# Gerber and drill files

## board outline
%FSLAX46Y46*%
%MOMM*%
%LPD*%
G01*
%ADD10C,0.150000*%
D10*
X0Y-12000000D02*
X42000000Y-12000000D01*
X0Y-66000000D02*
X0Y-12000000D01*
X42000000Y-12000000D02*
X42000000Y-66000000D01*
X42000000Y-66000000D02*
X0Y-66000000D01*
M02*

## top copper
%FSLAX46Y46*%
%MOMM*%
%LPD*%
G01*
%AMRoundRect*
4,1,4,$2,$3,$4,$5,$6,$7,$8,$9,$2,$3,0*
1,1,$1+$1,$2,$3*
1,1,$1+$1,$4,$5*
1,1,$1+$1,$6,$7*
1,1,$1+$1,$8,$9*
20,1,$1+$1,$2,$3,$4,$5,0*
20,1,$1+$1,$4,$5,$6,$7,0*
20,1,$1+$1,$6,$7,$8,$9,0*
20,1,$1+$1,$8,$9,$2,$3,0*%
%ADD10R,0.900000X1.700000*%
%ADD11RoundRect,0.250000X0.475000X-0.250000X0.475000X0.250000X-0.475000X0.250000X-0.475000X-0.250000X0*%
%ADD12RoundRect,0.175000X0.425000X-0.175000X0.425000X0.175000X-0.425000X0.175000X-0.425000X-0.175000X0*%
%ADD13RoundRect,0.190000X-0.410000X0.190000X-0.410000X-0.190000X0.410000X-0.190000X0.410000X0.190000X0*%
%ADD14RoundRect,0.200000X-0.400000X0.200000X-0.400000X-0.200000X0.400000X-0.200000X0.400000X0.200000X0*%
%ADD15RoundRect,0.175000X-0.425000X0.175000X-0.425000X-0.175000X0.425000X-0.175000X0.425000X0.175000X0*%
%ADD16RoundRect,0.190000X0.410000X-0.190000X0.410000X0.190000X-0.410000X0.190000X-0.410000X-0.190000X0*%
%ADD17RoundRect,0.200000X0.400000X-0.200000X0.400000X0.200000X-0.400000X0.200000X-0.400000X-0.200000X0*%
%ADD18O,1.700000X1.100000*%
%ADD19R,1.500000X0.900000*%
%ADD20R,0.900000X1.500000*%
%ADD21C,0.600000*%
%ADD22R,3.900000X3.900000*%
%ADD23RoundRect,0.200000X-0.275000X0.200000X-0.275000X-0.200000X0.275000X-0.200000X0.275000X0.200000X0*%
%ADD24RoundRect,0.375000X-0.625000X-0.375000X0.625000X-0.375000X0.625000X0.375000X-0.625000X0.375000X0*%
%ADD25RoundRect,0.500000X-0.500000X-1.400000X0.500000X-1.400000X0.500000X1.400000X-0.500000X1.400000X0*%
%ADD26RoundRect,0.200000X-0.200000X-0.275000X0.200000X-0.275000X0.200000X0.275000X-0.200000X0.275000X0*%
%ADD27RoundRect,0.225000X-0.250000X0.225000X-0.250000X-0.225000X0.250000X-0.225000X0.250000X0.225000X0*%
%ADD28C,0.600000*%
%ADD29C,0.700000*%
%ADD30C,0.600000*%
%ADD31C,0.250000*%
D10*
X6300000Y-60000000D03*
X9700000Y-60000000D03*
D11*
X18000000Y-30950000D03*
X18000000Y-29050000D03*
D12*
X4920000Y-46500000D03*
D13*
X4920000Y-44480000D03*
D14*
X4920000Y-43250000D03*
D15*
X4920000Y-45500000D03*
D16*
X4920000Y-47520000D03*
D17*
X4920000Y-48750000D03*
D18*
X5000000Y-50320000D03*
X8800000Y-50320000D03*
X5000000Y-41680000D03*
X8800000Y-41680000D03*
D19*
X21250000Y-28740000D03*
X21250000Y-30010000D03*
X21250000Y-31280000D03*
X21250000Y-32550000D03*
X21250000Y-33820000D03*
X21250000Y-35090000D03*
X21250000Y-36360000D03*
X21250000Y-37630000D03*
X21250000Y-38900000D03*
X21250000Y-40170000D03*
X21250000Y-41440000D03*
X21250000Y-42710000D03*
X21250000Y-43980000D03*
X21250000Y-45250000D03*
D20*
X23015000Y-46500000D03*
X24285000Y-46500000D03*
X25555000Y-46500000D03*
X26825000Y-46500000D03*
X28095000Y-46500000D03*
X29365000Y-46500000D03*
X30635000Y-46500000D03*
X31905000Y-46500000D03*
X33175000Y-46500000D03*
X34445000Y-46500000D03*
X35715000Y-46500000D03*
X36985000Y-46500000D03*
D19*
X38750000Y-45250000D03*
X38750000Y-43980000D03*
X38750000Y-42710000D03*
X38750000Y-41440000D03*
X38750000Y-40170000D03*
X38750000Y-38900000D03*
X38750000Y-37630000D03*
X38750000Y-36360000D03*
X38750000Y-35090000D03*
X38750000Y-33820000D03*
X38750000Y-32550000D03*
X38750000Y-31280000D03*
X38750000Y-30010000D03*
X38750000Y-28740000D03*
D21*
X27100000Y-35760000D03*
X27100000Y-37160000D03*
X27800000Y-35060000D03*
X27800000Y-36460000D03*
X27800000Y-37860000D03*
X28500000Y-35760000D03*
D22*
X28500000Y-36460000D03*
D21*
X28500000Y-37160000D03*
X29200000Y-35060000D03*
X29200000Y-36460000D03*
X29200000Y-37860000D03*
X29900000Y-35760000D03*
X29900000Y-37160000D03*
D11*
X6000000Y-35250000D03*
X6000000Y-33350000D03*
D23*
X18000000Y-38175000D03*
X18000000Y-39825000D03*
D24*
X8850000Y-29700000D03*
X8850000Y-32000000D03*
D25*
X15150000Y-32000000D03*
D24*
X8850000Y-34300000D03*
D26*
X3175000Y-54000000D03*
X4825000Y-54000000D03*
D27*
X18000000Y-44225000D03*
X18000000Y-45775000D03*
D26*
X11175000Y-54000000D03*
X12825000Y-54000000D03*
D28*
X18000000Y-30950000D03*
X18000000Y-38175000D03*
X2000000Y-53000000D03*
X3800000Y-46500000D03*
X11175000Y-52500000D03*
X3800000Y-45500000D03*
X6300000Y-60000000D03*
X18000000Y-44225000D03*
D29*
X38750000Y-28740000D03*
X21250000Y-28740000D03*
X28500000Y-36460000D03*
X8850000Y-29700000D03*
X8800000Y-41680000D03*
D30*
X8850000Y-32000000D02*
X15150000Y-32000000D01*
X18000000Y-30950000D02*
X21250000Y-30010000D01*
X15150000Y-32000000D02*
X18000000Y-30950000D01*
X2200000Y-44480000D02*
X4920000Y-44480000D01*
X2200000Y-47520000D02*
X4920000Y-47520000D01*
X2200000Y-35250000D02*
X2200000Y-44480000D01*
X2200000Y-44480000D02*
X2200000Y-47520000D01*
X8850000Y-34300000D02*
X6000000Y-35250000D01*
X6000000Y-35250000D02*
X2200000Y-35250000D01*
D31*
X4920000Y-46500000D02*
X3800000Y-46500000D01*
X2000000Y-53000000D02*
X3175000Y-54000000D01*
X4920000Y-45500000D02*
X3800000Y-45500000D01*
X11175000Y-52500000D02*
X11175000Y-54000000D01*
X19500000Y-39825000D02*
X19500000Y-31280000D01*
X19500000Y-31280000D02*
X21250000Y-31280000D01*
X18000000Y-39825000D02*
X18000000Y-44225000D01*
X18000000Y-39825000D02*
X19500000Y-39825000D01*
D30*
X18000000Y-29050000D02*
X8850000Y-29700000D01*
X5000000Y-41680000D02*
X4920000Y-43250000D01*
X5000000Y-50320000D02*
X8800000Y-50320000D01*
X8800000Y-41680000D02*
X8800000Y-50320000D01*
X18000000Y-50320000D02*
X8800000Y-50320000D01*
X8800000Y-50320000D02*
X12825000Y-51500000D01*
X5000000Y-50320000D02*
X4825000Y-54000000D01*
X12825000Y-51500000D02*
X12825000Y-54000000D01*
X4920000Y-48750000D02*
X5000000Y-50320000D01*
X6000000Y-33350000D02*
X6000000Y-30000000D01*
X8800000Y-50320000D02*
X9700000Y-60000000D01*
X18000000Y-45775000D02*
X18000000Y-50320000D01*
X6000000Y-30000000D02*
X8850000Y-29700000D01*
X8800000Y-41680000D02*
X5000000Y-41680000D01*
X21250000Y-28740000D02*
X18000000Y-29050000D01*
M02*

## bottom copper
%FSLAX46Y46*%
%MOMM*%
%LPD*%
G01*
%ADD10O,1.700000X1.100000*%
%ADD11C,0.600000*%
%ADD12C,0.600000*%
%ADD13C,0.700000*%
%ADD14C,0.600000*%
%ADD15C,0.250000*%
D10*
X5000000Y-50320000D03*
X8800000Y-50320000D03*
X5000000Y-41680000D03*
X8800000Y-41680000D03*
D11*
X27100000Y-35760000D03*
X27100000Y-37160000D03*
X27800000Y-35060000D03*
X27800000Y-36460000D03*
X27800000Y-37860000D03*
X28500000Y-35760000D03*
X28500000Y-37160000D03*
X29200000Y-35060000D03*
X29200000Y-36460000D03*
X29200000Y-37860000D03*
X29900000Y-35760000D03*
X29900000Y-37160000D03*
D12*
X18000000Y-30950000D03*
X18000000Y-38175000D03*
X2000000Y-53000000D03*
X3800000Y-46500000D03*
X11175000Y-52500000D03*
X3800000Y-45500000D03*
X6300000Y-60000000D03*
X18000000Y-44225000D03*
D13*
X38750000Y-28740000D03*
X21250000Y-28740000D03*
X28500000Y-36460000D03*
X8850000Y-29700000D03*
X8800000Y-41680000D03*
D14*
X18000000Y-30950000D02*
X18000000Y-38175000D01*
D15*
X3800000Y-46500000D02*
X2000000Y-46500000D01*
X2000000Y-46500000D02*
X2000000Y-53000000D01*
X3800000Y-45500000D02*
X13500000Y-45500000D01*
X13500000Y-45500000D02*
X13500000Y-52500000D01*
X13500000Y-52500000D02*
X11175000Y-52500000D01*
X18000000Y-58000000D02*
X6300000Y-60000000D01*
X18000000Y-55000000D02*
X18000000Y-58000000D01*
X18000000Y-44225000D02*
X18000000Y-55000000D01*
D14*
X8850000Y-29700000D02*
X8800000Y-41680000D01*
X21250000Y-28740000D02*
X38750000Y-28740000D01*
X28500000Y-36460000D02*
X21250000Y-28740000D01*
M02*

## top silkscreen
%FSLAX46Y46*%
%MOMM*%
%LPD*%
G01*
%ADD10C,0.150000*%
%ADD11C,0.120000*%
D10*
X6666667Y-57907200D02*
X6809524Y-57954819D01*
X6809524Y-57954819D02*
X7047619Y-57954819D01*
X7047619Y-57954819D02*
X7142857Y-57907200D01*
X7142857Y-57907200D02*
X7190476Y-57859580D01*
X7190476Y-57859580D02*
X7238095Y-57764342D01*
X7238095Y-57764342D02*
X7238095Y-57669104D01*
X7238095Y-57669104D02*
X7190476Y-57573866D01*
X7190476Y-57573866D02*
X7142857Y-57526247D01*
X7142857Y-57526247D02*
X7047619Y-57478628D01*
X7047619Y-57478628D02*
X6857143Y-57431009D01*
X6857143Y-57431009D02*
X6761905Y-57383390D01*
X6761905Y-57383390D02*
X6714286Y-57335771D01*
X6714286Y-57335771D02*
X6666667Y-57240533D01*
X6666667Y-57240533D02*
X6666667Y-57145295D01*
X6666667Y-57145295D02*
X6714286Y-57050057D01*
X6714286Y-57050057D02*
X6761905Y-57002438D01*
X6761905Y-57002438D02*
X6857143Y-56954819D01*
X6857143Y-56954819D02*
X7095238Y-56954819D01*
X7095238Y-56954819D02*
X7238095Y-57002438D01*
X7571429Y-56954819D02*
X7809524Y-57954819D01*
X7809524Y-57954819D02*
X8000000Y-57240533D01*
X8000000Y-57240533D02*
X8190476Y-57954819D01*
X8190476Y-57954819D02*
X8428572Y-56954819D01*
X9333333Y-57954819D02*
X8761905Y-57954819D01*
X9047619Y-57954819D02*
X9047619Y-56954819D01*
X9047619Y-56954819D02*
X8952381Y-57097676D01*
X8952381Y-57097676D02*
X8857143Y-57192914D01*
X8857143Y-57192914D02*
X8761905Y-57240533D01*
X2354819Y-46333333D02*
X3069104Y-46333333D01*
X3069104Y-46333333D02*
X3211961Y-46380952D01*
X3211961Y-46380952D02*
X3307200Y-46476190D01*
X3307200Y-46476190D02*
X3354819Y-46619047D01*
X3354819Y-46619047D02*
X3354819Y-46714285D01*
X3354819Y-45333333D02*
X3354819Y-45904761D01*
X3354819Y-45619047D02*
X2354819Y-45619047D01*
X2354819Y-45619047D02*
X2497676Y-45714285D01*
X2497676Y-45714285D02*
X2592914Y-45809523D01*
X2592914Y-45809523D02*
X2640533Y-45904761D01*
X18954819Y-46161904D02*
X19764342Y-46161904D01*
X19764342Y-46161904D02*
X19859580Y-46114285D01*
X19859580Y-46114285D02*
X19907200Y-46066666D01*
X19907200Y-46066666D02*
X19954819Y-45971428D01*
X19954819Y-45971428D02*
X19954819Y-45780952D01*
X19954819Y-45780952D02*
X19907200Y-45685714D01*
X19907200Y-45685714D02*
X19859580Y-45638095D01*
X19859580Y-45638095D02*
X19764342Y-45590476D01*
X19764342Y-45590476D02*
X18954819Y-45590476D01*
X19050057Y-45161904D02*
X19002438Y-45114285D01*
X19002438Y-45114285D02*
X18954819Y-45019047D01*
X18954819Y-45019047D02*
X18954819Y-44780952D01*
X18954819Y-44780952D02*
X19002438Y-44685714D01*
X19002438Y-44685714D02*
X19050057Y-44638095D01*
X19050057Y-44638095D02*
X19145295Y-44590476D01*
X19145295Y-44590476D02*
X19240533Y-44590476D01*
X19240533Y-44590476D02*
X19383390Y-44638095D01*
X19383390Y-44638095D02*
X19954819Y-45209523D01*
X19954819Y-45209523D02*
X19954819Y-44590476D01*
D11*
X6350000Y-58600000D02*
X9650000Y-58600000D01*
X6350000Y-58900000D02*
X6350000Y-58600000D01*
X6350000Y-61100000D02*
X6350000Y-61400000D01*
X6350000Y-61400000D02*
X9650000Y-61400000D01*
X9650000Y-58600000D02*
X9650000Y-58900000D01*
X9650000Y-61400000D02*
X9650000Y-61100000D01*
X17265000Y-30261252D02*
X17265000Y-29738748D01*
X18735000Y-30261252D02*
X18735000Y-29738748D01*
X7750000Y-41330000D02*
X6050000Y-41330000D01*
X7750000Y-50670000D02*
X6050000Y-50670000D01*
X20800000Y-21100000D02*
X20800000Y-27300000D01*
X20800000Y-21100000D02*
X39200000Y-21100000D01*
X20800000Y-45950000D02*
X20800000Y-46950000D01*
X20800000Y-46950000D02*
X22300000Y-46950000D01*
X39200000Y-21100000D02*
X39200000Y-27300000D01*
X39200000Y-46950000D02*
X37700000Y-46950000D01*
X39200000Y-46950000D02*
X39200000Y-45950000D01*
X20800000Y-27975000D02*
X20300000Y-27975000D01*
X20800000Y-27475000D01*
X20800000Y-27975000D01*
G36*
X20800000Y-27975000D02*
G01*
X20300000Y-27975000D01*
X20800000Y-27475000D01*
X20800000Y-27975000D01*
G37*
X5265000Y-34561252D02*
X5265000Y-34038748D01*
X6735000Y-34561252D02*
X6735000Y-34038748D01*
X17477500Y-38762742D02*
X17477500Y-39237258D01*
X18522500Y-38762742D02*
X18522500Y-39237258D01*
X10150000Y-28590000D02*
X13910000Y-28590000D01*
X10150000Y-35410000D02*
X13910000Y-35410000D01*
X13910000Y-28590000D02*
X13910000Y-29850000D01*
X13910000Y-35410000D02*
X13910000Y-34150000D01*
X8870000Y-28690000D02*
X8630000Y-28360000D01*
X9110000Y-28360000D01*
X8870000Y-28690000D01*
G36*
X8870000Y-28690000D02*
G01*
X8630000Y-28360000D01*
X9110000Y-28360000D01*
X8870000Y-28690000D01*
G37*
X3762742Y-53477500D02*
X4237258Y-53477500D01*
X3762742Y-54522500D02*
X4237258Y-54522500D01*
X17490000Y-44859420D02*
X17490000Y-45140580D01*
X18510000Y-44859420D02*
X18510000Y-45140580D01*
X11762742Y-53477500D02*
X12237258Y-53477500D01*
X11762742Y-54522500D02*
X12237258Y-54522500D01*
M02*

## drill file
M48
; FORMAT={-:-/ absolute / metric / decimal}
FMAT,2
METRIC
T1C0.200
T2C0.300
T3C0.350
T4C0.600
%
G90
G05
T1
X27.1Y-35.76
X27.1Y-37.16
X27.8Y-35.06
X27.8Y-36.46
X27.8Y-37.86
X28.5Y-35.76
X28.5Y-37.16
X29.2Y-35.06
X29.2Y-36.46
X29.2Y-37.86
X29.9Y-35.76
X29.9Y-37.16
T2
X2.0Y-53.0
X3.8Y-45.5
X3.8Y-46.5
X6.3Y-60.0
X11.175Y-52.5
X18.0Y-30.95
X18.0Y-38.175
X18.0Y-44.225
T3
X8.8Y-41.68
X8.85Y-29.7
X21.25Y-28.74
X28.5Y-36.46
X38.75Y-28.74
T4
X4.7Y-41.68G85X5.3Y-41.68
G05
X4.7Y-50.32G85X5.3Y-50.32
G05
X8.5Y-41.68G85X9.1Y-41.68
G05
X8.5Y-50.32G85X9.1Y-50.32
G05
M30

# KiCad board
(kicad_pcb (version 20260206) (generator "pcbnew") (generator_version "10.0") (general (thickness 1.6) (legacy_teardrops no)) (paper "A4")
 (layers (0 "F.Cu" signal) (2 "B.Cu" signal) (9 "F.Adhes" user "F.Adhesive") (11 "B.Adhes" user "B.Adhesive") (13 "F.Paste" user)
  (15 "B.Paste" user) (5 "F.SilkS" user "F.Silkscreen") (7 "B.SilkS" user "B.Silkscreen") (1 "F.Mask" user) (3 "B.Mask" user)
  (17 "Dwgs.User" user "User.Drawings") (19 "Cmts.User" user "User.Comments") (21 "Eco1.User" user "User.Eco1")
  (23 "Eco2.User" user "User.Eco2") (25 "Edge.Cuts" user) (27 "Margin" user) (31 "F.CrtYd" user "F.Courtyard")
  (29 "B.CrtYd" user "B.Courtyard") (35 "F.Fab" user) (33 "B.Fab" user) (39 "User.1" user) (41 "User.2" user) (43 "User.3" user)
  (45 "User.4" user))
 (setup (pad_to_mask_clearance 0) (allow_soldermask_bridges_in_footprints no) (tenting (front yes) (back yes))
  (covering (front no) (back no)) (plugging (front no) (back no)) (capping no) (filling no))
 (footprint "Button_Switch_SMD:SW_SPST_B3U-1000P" (layer "F.Cu") (at 8 60)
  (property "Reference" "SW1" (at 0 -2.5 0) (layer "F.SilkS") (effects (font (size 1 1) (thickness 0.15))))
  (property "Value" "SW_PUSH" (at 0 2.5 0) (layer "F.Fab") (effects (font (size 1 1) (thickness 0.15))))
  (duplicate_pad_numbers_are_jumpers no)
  (fp_line (start -1.65 -1.4) (end 1.65 -1.4) (stroke (width 0.12) (type solid)) (layer "F.SilkS"))
  (fp_line (start -1.65 -1.1) (end -1.65 -1.4) (stroke (width 0.12) (type solid)) (layer "F.SilkS"))
  (fp_line (start -1.65 1.1) (end -1.65 1.4) (stroke (width 0.12) (type solid)) (layer "F.SilkS"))
  (fp_line (start -1.65 1.4) (end 1.65 1.4) (stroke (width 0.12) (type solid)) (layer "F.SilkS"))
  (fp_line (start 1.65 -1.4) (end 1.65 -1.1) (stroke (width 0.12) (type solid)) (layer "F.SilkS"))
  (fp_line (start 1.65 1.4) (end 1.65 1.1) (stroke (width 0.12) (type solid)) (layer "F.SilkS"))
  (pad "1" smd rect (at -1.7 0) (size 0.9 1.7) (layers "F.Cu" "F.Mask" "F.Paste") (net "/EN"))
  (pad "2" smd rect (at 1.7 0) (size 0.9 1.7) (layers "F.Cu" "F.Mask" "F.Paste") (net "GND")))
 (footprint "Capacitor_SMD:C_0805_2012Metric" (layer "F.Cu") (at 18 30 90)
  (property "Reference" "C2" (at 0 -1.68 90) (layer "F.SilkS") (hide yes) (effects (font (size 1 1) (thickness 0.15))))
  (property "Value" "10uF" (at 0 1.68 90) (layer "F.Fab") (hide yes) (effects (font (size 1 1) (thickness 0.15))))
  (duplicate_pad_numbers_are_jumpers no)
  (fp_line (start -0.261252 -0.735) (end 0.261252 -0.735) (stroke (width 0.12) (type solid)) (layer "F.SilkS"))
  (fp_line (start -0.261252 0.735) (end 0.261252 0.735) (stroke (width 0.12) (type solid)) (layer "F.SilkS"))
  (pad "1" smd roundrect (at -0.95 0 90) (size 1 1.45) (layers "F.Cu" "F.Mask" "F.Paste") (roundrect_rratio 0.25) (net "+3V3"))
  (pad "2" smd roundrect (at 0.95 0 90) (size 1 1.45) (layers "F.Cu" "F.Mask" "F.Paste") (roundrect_rratio 0.25) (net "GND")))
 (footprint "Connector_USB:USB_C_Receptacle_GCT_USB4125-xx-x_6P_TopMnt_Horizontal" (layer "F.Cu") (at 8 46 90)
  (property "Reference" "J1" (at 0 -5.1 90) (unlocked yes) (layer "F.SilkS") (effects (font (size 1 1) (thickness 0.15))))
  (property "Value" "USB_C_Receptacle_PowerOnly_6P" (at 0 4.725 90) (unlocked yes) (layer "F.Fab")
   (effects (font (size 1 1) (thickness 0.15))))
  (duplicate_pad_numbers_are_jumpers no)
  (fp_line (start 4.67 -0.25) (end 4.67 -1.95) (stroke (width 0.12) (type solid)) (layer "F.SilkS"))
  (fp_line (start -4.67 -0.25) (end -4.67 -1.95) (stroke (width 0.12) (type solid)) (layer "F.SilkS"))
  (pad "A5" smd roundrect (at -0.5 -3.08 90) (size 0.7 1.2) (layers "F.Cu" "F.Mask" "F.Paste") (roundrect_rratio 0.25) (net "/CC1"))
  (pad "A9" smd roundrect (at 1.52 -3.08 270) (size 0.76 1.2) (layers "F.Cu" "F.Mask" "F.Paste") (roundrect_rratio 0.25) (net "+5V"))
  (pad "A12" smd roundrect (at 2.75 -3.08 270) (size 0.8 1.2) (layers "F.Cu" "F.Mask" "F.Paste") (roundrect_rratio 0.25) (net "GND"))
  (pad "B5" smd roundrect (at 0.5 -3.08 270) (size 0.7 1.2) (layers "F.Cu" "F.Mask" "F.Paste") (roundrect_rratio 0.25) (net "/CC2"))
  (pad "B9" smd roundrect (at -1.52 -3.08 90) (size 0.76 1.2) (layers "F.Cu" "F.Mask" "F.Paste") (roundrect_rratio 0.25) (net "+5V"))
  (pad "B12" smd roundrect (at -2.75 -3.08 90) (size 0.8 1.2) (layers "F.Cu" "F.Mask" "F.Paste") (roundrect_rratio 0.25) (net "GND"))
  (pad "SH" thru_hole oval (at -4.32 -3 90) (size 1.1 1.7) (drill oval 0.6 1.2) (layers "*.Cu" "*.Mask" "F.Paste") (remove_unused_layers no)
   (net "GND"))
  (pad "SH" thru_hole oval (at -4.32 0.8 90) (size 1.1 1.7) (drill oval 0.6 1.2) (layers "*.Cu" "*.Mask" "F.Paste")
   (remove_unused_layers no) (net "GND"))
  (pad "SH" thru_hole oval (at 4.32 -3 90) (size 1.1 1.7) (drill oval 0.6 1.2) (layers "*.Cu" "*.Mask" "F.Paste") (remove_unused_layers no)
   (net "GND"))
  (pad "SH" thru_hole oval (at 4.32 0.8 90) (size 1.1 1.7) (drill oval 0.6 1.2) (layers "*.Cu" "*.Mask" "F.Paste") (remove_unused_layers no)
   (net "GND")))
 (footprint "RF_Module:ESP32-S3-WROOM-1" (layer "F.Cu") (at 30 34)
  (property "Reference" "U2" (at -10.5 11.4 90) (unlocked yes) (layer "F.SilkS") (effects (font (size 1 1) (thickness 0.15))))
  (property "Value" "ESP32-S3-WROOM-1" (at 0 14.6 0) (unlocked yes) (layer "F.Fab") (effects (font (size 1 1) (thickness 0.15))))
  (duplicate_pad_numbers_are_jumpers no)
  (fp_line (start -9.2 -12.9) (end -9.2 -6.7) (stroke (width 0.12) (type solid)) (layer "F.SilkS"))
  (fp_line (start -9.2 -12.9) (end 9.2 -12.9) (stroke (width 0.12) (type solid)) (layer "F.SilkS"))
  (fp_line (start -9.2 11.95) (end -9.2 12.95) (stroke (width 0.12) (type solid)) (layer "F.SilkS"))
  (fp_line (start -9.2 12.95) (end -7.7 12.95) (stroke (width 0.12) (type solid)) (layer "F.SilkS"))
  (fp_line (start 9.2 -12.9) (end 9.2 -6.7) (stroke (width 0.12) (type solid)) (layer "F.SilkS"))
  (fp_line (start 9.2 12.95) (end 7.7 12.95) (stroke (width 0.12) (type solid)) (layer "F.SilkS"))
  (fp_line (start 9.2 12.95) (end 9.2 11.95) (stroke (width 0.12) (type solid)) (layer "F.SilkS"))
  (fp_poly
   (pts (xy -9.2 -6.025) (xy -9.7 -6.025) (xy -9.2 -6.525) (xy -9.2 -6.025)) (stroke (width 0.12) (type solid)) (fill yes) (layer "F.SilkS"))
  (pad "" smd rect (at -2.9 1.06) (size 0.9 0.9) (layers "F.Paste"))
  (pad "" smd rect (at -2.9 2.46 270) (size 0.9 0.9) (layers "F.Paste"))
  (pad "" smd rect (at -2.9 3.86) (size 0.9 0.9) (layers "F.Paste"))
  (pad "" smd rect (at -1.5 1.06 270) (size 0.9 0.9) (layers "F.Paste"))
  (pad "" smd rect (at -1.5 2.46 270) (size 0.9 0.9) (layers "F.Paste"))
  (pad "" smd rect (at -1.5 3.86 270) (size 0.9 0.9) (layers "F.Paste"))
  (pad "" smd rect (at -0.1 1.06 270) (size 0.9 0.9) (layers "F.Paste"))
  (pad "" smd rect (at -0.1 2.46 270) (size 0.9 0.9) (layers "F.Paste"))
  (pad "" smd rect (at -0.1 3.86 270) (size 0.9 0.9) (layers "F.Paste"))
  (pad "1" smd rect (at -8.75 -5.26) (size 1.5 0.9) (layers "F.Cu" "F.Mask" "F.Paste") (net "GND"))
  (pad "2" smd rect (at -8.75 -3.99) (size 1.5 0.9) (layers "F.Cu" "F.Mask" "F.Paste") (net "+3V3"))
  (pad "3" smd rect (at -8.75 -2.72) (size 1.5 0.9) (layers "F.Cu" "F.Mask" "F.Paste") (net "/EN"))
  (pad "4" smd rect (at -8.75 -1.45) (size 1.5 0.9) (layers "F.Cu" "F.Mask" "F.Paste"))
  (pad "5" smd rect (at -8.75 -0.18) (size 1.5 0.9) (layers "F.Cu" "F.Mask" "F.Paste"))
  (pad "6" smd rect (at -8.75 1.09) (size 1.5 0.9) (layers "F.Cu" "F.Mask" "F.Paste"))
  (pad "7" smd rect (at -8.75 2.36) (size 1.5 0.9) (layers "F.Cu" "F.Mask" "F.Paste"))
  (pad "8" smd rect (at -8.75 3.63) (size 1.5 0.9) (layers "F.Cu" "F.Mask" "F.Paste"))
  (pad "9" smd rect (at -8.75 4.9) (size 1.5 0.9) (layers "F.Cu" "F.Mask" "F.Paste"))
  (pad "10" smd rect (at -8.75 6.17) (size 1.5 0.9) (layers "F.Cu" "F.Mask" "F.Paste"))
  (pad "11" smd rect (at -8.75 7.44) (size 1.5 0.9) (layers "F.Cu" "F.Mask" "F.Paste"))
  (pad "12" smd rect (at -8.75 8.71) (size 1.5 0.9) (layers "F.Cu" "F.Mask" "F.Paste"))
  (pad "13" smd rect (at -8.75 9.98) (size 1.5 0.9) (layers "F.Cu" "F.Mask" "F.Paste"))
  (pad "14" smd rect (at -8.75 11.25 180) (size 1.5 0.9) (layers "F.Cu" "F.Mask" "F.Paste"))
  (pad "15" smd rect (at -6.985 12.5 270) (size 1.5 0.9) (layers "F.Cu" "F.Mask" "F.Paste"))
  (pad "16" smd rect (at -5.715 12.5 270) (size 1.5 0.9) (layers "F.Cu" "F.Mask" "F.Paste"))
  (pad "17" smd rect (at -4.445 12.5 270) (size 1.5 0.9) (layers "F.Cu" "F.Mask" "F.Paste"))
  (pad "18" smd rect (at -3.175 12.5 270) (size 1.5 0.9) (layers "F.Cu" "F.Mask" "F.Paste"))
  (pad "19" smd rect (at -1.905 12.5 270) (size 1.5 0.9) (layers "F.Cu" "F.Mask" "F.Paste"))
  (pad "20" smd rect (at -0.635 12.5 270) (size 1.5 0.9) (layers "F.Cu" "F.Mask" "F.Paste"))
  (pad "21" smd rect (at 0.635 12.5 270) (size 1.5 0.9) (layers "F.Cu" "F.Mask" "F.Paste"))
  (pad "22" smd rect (at 1.905 12.5 270) (size 1.5 0.9) (layers "F.Cu" "F.Mask" "F.Paste"))
  (pad "23" smd rect (at 3.175 12.5 270) (size 1.5 0.9) (layers "F.Cu" "F.Mask" "F.Paste"))
  (pad "24" smd rect (at 4.445 12.5 270) (size 1.5 0.9) (layers "F.Cu" "F.Mask" "F.Paste"))
  (pad "25" smd rect (at 5.715 12.5 270) (size 1.5 0.9) (layers "F.Cu" "F.Mask" "F.Paste"))
  (pad "26" smd rect (at 6.985 12.5 270) (size 1.5 0.9) (layers "F.Cu" "F.Mask" "F.Paste"))
  (pad "27" smd rect (at 8.75 11.25) (size 1.5 0.9) (layers "F.Cu" "F.Mask" "F.Paste"))
  (pad "28" smd rect (at 8.75 9.98) (size 1.5 0.9) (layers "F.Cu" "F.Mask" "F.Paste"))
  (pad "29" smd rect (at 8.75 8.71) (size 1.5 0.9) (layers "F.Cu" "F.Mask" "F.Paste"))
  (pad "30" smd rect (at 8.75 7.44) (size 1.5 0.9) (layers "F.Cu" "F.Mask" "F.Paste"))
  (pad "31" smd rect (at 8.75 6.17) (size 1.5 0.9) (layers "F.Cu" "F.Mask" "F.Paste"))
  (pad "32" smd rect (at 8.75 4.9) (size 1.5 0.9) (layers "F.Cu" "F.Mask" "F.Paste"))
  (pad "33" smd rect (at 8.75 3.63) (size 1.5 0.9) (layers "F.Cu" "F.Mask" "F.Paste"))
  (pad "34" smd rect (at 8.75 2.36) (size 1.5 0.9) (layers "F.Cu" "F.Mask" "F.Paste"))
  (pad "35" smd rect (at 8.75 1.09) (size 1.5 0.9) (layers "F.Cu" "F.Mask" "F.Paste"))
  (pad "36" smd rect (at 8.75 -0.18) (size 1.5 0.9) (layers "F.Cu" "F.Mask" "F.Paste"))
  (pad "37" smd rect (at 8.75 -1.45) (size 1.5 0.9) (layers "F.Cu" "F.Mask" "F.Paste"))
  (pad "38" smd rect (at 8.75 -2.72) (size 1.5 0.9) (layers "F.Cu" "F.Mask" "F.Paste"))
  (pad "39" smd rect (at 8.75 -3.99) (size 1.5 0.9) (layers "F.Cu" "F.Mask" "F.Paste"))
  (pad "40" smd rect (at 8.75 -5.26) (size 1.5 0.9) (layers "F.Cu" "F.Mask" "F.Paste") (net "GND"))
  (pad "41" thru_hole circle (at -2.9 1.76 90) (size 0.6 0.6) (drill 0.2) (layers "*.Cu" "F.Mask") (remove_unused_layers no) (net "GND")
   (zone_connect 2))
  (pad "41" thru_hole circle (at -2.9 3.16) (size 0.6 0.6) (drill 0.2) (layers "*.Cu" "F.Mask") (remove_unused_layers no) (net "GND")
   (zone_connect 2))
  (pad "41" thru_hole circle (at -2.2 1.06) (size 0.6 0.6) (drill 0.2) (layers "*.Cu" "F.Mask") (remove_unused_layers no) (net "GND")
   (zone_connect 2))
  (pad "41" thru_hole circle (at -2.2 2.46) (size 0.6 0.6) (drill 0.2) (layers "*.Cu" "F.Mask") (remove_unused_layers no) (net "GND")
   (zone_connect 2))
  (pad "41" thru_hole circle (at -2.2 3.86) (size 0.6 0.6) (drill 0.2) (layers "*.Cu" "F.Mask") (remove_unused_layers no) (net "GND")
   (zone_connect 2))
  (pad "41" thru_hole circle (at -1.5 1.76) (size 0.6 0.6) (drill 0.2) (layers "*.Cu" "F.Mask") (remove_unused_layers no) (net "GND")
   (zone_connect 2))
  (pad "41" smd rect (at -1.5 2.46 270) (size 3.9 3.9) (layers "F.Cu" "F.Mask") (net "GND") (zone_connect 2))
  (pad "41" thru_hole circle (at -1.5 3.16) (size 0.6 0.6) (drill 0.2) (layers "*.Cu" "F.Mask") (remove_unused_layers no) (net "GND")
   (zone_connect 2))
  (pad "41" thru_hole circle (at -0.8 1.06) (size 0.6 0.6) (drill 0.2) (layers "*.Cu" "F.Mask") (remove_unused_layers no) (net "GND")
   (zone_connect 2))
  (pad "41" thru_hole circle (at -0.8 2.46) (size 0.6 0.6) (drill 0.2) (layers "*.Cu" "F.Mask") (remove_unused_layers no) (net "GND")
   (zone_connect 2))
  (pad "41" thru_hole circle (at -0.8 3.86) (size 0.6 0.6) (drill 0.2) (layers "*.Cu" "F.Mask") (remove_unused_layers no) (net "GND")
   (zone_connect 2))
  (pad "41" thru_hole circle (at -0.1 1.76) (size 0.6 0.6) (drill 0.2) (layers "*.Cu" "F.Mask") (remove_unused_layers no) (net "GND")
   (zone_connect 2))
  (pad "41" thru_hole circle (at -0.1 3.16) (size 0.6 0.6) (drill 0.2) (layers "*.Cu" "F.Mask") (remove_unused_layers no) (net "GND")
   (zone_connect 2))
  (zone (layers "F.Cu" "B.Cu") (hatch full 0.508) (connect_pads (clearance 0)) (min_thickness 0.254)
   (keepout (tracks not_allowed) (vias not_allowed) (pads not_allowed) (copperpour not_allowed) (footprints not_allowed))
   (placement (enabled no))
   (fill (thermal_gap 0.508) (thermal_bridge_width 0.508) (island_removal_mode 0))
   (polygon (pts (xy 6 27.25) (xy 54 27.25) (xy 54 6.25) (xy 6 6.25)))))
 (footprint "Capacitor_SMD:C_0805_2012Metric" (layer "F.Cu") (at 6 34.3 90)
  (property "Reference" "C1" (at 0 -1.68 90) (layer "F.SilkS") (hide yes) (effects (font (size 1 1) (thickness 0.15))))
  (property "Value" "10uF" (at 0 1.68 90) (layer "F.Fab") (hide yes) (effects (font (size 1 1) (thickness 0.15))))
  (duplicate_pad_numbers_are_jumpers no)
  (fp_line (start -0.261252 -0.735) (end 0.261252 -0.735) (stroke (width 0.12) (type solid)) (layer "F.SilkS"))
  (fp_line (start -0.261252 0.735) (end 0.261252 0.735) (stroke (width 0.12) (type solid)) (layer "F.SilkS"))
  (pad "1" smd roundrect (at -0.95 0 90) (size 1 1.45) (layers "F.Cu" "F.Mask" "F.Paste") (roundrect_rratio 0.25) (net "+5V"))
  (pad "2" smd roundrect (at 0.95 0 90) (size 1 1.45) (layers "F.Cu" "F.Mask" "F.Paste") (roundrect_rratio 0.25) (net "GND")))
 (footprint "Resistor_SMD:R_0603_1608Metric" (layer "F.Cu") (at 18 39 -90)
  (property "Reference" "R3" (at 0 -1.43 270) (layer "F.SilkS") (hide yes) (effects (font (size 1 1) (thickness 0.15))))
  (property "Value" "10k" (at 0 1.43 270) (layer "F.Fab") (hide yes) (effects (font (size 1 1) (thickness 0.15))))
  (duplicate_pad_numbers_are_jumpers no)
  (fp_line (start -0.237258 0.5225) (end 0.237258 0.5225) (stroke (width 0.12) (type solid)) (layer "F.SilkS"))
  (fp_line (start -0.237258 -0.5225) (end 0.237258 -0.5225) (stroke (width 0.12) (type solid)) (layer "F.SilkS"))
  (pad "1" smd roundrect (at -0.825 0 270) (size 0.8 0.95) (layers "F.Cu" "F.Mask" "F.Paste") (roundrect_rratio 0.25) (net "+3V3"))
  (pad "2" smd roundrect (at 0.825 0 270) (size 0.8 0.95) (layers "F.Cu" "F.Mask" "F.Paste") (roundrect_rratio 0.25) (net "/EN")))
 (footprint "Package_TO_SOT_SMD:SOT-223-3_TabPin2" (layer "F.Cu") (at 12 32)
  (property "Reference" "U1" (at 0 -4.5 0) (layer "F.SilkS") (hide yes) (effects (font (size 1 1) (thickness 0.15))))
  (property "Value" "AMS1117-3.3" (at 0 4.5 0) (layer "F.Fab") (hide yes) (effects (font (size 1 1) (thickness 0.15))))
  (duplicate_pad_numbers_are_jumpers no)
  (fp_line (start -1.85 -3.41) (end 1.91 -3.41) (stroke (width 0.12) (type solid)) (layer "F.SilkS"))
  (fp_line (start -1.85 3.41) (end 1.91 3.41) (stroke (width 0.12) (type solid)) (layer "F.SilkS"))
  (fp_line (start 1.91 -3.41) (end 1.91 -2.15) (stroke (width 0.12) (type solid)) (layer "F.SilkS"))
  (fp_line (start 1.91 3.41) (end 1.91 2.15) (stroke (width 0.12) (type solid)) (layer "F.SilkS"))
  (fp_poly
   (pts (xy -3.13 -3.31) (xy -3.37 -3.64) (xy -2.89 -3.64) (xy -3.13 -3.31)) (stroke (width 0.12) (type solid)) (fill yes) (layer "F.SilkS"))
  (pad "1" smd roundrect (at -3.15 -2.3) (size 2 1.5) (layers "F.Cu" "F.Mask" "F.Paste") (roundrect_rratio 0.25) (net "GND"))
  (pad "2" smd roundrect (at -3.15 0) (size 2 1.5) (layers "F.Cu" "F.Mask" "F.Paste") (roundrect_rratio 0.25) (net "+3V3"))
  (pad "2" smd roundrect (at 3.15 0) (size 2 3.8) (layers "F.Cu" "F.Mask" "F.Paste") (roundrect_rratio 0.25) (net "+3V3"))
  (pad "3" smd roundrect (at -3.15 2.3) (size 2 1.5) (layers "F.Cu" "F.Mask" "F.Paste") (roundrect_rratio 0.25) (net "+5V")))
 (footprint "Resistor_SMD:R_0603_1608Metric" (layer "F.Cu") (at 4 54)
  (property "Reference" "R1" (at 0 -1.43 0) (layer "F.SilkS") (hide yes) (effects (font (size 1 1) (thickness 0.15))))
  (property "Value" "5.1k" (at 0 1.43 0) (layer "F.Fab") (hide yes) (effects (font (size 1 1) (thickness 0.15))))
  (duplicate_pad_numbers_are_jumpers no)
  (fp_line (start -0.237258 -0.5225) (end 0.237258 -0.5225) (stroke (width 0.12) (type solid)) (layer "F.SilkS"))
  (fp_line (start -0.237258 0.5225) (end 0.237258 0.5225) (stroke (width 0.12) (type solid)) (layer "F.SilkS"))
  (pad "1" smd roundrect (at -0.825 0) (size 0.8 0.95) (layers "F.Cu" "F.Mask" "F.Paste") (roundrect_rratio 0.25) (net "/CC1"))
  (pad "2" smd roundrect (at 0.825 0) (size 0.8 0.95) (layers "F.Cu" "F.Mask" "F.Paste") (roundrect_rratio 0.25) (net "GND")))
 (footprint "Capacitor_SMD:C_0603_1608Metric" (layer "F.Cu") (at 18 45 -90)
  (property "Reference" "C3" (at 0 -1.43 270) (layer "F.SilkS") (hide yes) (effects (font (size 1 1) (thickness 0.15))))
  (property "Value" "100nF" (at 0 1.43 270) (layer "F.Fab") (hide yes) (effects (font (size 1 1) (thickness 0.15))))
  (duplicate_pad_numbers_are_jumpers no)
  (fp_line (start -0.14058 0.51) (end 0.14058 0.51) (stroke (width 0.12) (type solid)) (layer "F.SilkS"))
  (fp_line (start -0.14058 -0.51) (end 0.14058 -0.51) (stroke (width 0.12) (type solid)) (layer "F.SilkS"))
  (pad "1" smd roundrect (at -0.775 0 270) (size 0.9 0.95) (layers "F.Cu" "F.Mask" "F.Paste") (roundrect_rratio 0.25) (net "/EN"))
  (pad "2" smd roundrect (at 0.775 0 270) (size 0.9 0.95) (layers "F.Cu" "F.Mask" "F.Paste") (roundrect_rratio 0.25) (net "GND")))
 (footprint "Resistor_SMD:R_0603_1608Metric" (layer "F.Cu") (at 12 54)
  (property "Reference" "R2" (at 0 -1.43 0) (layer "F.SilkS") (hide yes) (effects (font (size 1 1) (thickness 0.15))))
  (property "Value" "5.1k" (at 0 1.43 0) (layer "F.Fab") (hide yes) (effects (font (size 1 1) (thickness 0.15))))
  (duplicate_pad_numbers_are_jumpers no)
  (fp_line (start -0.237258 -0.5225) (end 0.237258 -0.5225) (stroke (width 0.12) (type solid)) (layer "F.SilkS"))
  (fp_line (start -0.237258 0.5225) (end 0.237258 0.5225) (stroke (width 0.12) (type solid)) (layer "F.SilkS"))
  (pad "1" smd roundrect (at -0.825 0) (size 0.8 0.95) (layers "F.Cu" "F.Mask" "F.Paste") (roundrect_rratio 0.25) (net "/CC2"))
  (pad "2" smd roundrect (at 0.825 0) (size 0.8 0.95) (layers "F.Cu" "F.Mask" "F.Paste") (roundrect_rratio 0.25) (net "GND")))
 (gr_line (start 0 12) (end 42 12) (stroke (width 0.15) (type default)) (layer "Edge.Cuts"))
 (gr_line (start 0 66) (end 0 12) (stroke (width 0.15) (type default)) (layer "Edge.Cuts"))
 (gr_line (start 42 12) (end 42 66) (stroke (width 0.15) (type default)) (layer "Edge.Cuts"))
 (gr_line (start 42 66) (end 0 66) (stroke (width 0.15) (type default)) (layer "Edge.Cuts"))
 (segment (start 8.85 32) (end 15.15 32) (width 0.6) (layer "F.Cu") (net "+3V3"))
 (segment (start 18 30.95) (end 21.25 30.01) (width 0.6) (layer "F.Cu") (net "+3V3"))
 (segment (start 15.15 32) (end 18 30.95) (width 0.6) (layer "F.Cu") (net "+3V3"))
 (via (at 18 30.95) (size 0.6) (drill 0.3) (layers "F.Cu" "B.Cu") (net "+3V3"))
 (via (at 18 38.175) (size 0.6) (drill 0.3) (layers "F.Cu" "B.Cu") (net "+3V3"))
 (segment (start 18 30.95) (end 18 38.175) (width 0.6) (layer "B.Cu") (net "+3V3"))
 (segment (start 2.2 44.48) (end 4.92 44.48) (width 0.6) (layer "F.Cu") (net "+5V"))
 (segment (start 2.2 47.52) (end 4.92 47.52) (width 0.6) (layer "F.Cu") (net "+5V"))
 (segment (start 2.2 35.25) (end 2.2 44.48) (width 0.6) (layer "F.Cu") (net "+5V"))
 (segment (start 2.2 44.48) (end 2.2 47.52) (width 0.6) (layer "F.Cu") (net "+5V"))
 (segment (start 8.85 34.3) (end 6 35.25) (width 0.6) (layer "F.Cu") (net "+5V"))
 (segment (start 6 35.25) (end 2.2 35.25) (width 0.6) (layer "F.Cu") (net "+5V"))
 (segment (start 4.92 46.5) (end 3.8 46.5) (width 0.25) (layer "F.Cu") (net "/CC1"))
 (segment (start 2 53) (end 3.175 54) (width 0.25) (layer "F.Cu") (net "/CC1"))
 (via (at 2 53) (size 0.6) (drill 0.3) (layers "F.Cu" "B.Cu") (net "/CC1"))
 (via (at 3.8 46.5) (size 0.6) (drill 0.3) (layers "F.Cu" "B.Cu") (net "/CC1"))
 (segment (start 3.8 46.5) (end 2 46.5) (width 0.25) (layer "B.Cu") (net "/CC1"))
 (segment (start 2 46.5) (end 2 53) (width 0.25) (layer "B.Cu") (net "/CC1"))
 (segment (start 4.92 45.5) (end 3.8 45.5) (width 0.25) (layer "F.Cu") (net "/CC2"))
 (segment (start 11.175 52.5) (end 11.175 54) (width 0.25) (layer "F.Cu") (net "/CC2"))
 (via (at 11.175 52.5) (size 0.6) (drill 0.3) (layers "F.Cu" "B.Cu") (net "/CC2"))
 (via (at 3.8 45.5) (size 0.6) (drill 0.3) (layers "F.Cu" "B.Cu") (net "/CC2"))
 (segment (start 3.8 45.5) (end 13.5 45.5) (width 0.25) (layer "B.Cu") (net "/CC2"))
 (segment (start 13.5 45.5) (end 13.5 52.5) (width 0.25) (layer "B.Cu") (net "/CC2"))
 (segment (start 13.5 52.5) (end 11.175 52.5) (width 0.25) (layer "B.Cu") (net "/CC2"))
 (segment (start 19.5 39.825) (end 19.5 31.28) (width 0.25) (layer "F.Cu") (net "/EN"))
 (segment (start 19.5 31.28) (end 21.25 31.28) (width 0.25) (layer "F.Cu") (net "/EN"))
 (segment (start 18 39.825) (end 18 44.225) (width 0.25) (layer "F.Cu") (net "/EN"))
 (segment (start 18 39.825) (end 19.5 39.825) (width 0.25) (layer "F.Cu") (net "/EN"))
 (via (at 6.3 60) (size 0.6) (drill 0.3) (layers "F.Cu" "B.Cu") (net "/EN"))
 (via (at 18 44.225) (size 0.6) (drill 0.3) (layers "F.Cu" "B.Cu") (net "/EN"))
 (segment (start 18 58) (end 6.3 60) (width 0.25) (layer "B.Cu") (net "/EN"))
 (segment (start 18 55) (end 18 58) (width 0.25) (layer "B.Cu") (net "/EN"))
 (segment (start 18 44.225) (end 18 55) (width 0.25) (layer "B.Cu") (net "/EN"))
 (segment (start 18 29.05) (end 8.85 29.7) (width 0.6) (layer "F.Cu") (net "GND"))
 (segment (start 5 41.68) (end 4.92 43.25) (width 0.6) (layer "F.Cu") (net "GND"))
 (segment (start 5 50.32) (end 8.8 50.32) (width 0.6) (layer "F.Cu") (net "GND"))
 (segment (start 8.8 41.68) (end 8.8 50.32) (width 0.6) (layer "F.Cu") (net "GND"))
 (segment (start 18 50.32) (end 8.8 50.32) (width 0.6) (layer "F.Cu") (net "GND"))
 (segment (start 8.8 50.32) (end 12.825 51.5) (width 0.6) (layer "F.Cu") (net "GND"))
 (segment (start 5 50.32) (end 4.825 54) (width 0.6) (layer "F.Cu") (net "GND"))
 (segment (start 12.825 51.5) (end 12.825 54) (width 0.6) (layer "F.Cu") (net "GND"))
 (segment (start 4.92 48.75) (end 5 50.32) (width 0.6) (layer "F.Cu") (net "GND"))
 (segment (start 6 33.35) (end 6 30) (width 0.6) (layer "F.Cu") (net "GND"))
 (segment (start 8.8 50.32) (end 9.7 60) (width 0.6) (layer "F.Cu") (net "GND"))
 (segment (start 18 45.775) (end 18 50.32) (width 0.6) (layer "F.Cu") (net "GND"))
 (segment (start 6 30) (end 8.85 29.7) (width 0.6) (layer "F.Cu") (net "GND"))
 (segment (start 8.8 41.68) (end 5 41.68) (width 0.6) (layer "F.Cu") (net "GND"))
 (segment (start 21.25 28.74) (end 18 29.05) (width 0.6) (layer "F.Cu") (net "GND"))
 (via (at 38.75 28.74) (size 0.7) (drill 0.35) (layers "F.Cu" "B.Cu") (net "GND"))
 (via (at 21.25 28.74) (size 0.7) (drill 0.35) (layers "F.Cu" "B.Cu") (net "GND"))
 (via (at 28.5 36.46) (size 0.7) (drill 0.35) (layers "F.Cu" "B.Cu") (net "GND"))
 (via (at 8.85 29.7) (size 0.7) (drill 0.35) (layers "F.Cu" "B.Cu") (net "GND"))
 (via (at 8.8 41.68) (size 0.7) (drill 0.35) (layers "F.Cu" "B.Cu") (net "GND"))
 (segment (start 8.85 29.7) (end 8.8 41.68) (width 0.6) (layer "B.Cu") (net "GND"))
 (segment (start 21.25 28.74) (end 38.75 28.74) (width 0.6) (layer "B.Cu") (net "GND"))
 (segment (start 28.5 36.46) (end 21.25 28.74) (width 0.6) (layer "B.Cu") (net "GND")))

